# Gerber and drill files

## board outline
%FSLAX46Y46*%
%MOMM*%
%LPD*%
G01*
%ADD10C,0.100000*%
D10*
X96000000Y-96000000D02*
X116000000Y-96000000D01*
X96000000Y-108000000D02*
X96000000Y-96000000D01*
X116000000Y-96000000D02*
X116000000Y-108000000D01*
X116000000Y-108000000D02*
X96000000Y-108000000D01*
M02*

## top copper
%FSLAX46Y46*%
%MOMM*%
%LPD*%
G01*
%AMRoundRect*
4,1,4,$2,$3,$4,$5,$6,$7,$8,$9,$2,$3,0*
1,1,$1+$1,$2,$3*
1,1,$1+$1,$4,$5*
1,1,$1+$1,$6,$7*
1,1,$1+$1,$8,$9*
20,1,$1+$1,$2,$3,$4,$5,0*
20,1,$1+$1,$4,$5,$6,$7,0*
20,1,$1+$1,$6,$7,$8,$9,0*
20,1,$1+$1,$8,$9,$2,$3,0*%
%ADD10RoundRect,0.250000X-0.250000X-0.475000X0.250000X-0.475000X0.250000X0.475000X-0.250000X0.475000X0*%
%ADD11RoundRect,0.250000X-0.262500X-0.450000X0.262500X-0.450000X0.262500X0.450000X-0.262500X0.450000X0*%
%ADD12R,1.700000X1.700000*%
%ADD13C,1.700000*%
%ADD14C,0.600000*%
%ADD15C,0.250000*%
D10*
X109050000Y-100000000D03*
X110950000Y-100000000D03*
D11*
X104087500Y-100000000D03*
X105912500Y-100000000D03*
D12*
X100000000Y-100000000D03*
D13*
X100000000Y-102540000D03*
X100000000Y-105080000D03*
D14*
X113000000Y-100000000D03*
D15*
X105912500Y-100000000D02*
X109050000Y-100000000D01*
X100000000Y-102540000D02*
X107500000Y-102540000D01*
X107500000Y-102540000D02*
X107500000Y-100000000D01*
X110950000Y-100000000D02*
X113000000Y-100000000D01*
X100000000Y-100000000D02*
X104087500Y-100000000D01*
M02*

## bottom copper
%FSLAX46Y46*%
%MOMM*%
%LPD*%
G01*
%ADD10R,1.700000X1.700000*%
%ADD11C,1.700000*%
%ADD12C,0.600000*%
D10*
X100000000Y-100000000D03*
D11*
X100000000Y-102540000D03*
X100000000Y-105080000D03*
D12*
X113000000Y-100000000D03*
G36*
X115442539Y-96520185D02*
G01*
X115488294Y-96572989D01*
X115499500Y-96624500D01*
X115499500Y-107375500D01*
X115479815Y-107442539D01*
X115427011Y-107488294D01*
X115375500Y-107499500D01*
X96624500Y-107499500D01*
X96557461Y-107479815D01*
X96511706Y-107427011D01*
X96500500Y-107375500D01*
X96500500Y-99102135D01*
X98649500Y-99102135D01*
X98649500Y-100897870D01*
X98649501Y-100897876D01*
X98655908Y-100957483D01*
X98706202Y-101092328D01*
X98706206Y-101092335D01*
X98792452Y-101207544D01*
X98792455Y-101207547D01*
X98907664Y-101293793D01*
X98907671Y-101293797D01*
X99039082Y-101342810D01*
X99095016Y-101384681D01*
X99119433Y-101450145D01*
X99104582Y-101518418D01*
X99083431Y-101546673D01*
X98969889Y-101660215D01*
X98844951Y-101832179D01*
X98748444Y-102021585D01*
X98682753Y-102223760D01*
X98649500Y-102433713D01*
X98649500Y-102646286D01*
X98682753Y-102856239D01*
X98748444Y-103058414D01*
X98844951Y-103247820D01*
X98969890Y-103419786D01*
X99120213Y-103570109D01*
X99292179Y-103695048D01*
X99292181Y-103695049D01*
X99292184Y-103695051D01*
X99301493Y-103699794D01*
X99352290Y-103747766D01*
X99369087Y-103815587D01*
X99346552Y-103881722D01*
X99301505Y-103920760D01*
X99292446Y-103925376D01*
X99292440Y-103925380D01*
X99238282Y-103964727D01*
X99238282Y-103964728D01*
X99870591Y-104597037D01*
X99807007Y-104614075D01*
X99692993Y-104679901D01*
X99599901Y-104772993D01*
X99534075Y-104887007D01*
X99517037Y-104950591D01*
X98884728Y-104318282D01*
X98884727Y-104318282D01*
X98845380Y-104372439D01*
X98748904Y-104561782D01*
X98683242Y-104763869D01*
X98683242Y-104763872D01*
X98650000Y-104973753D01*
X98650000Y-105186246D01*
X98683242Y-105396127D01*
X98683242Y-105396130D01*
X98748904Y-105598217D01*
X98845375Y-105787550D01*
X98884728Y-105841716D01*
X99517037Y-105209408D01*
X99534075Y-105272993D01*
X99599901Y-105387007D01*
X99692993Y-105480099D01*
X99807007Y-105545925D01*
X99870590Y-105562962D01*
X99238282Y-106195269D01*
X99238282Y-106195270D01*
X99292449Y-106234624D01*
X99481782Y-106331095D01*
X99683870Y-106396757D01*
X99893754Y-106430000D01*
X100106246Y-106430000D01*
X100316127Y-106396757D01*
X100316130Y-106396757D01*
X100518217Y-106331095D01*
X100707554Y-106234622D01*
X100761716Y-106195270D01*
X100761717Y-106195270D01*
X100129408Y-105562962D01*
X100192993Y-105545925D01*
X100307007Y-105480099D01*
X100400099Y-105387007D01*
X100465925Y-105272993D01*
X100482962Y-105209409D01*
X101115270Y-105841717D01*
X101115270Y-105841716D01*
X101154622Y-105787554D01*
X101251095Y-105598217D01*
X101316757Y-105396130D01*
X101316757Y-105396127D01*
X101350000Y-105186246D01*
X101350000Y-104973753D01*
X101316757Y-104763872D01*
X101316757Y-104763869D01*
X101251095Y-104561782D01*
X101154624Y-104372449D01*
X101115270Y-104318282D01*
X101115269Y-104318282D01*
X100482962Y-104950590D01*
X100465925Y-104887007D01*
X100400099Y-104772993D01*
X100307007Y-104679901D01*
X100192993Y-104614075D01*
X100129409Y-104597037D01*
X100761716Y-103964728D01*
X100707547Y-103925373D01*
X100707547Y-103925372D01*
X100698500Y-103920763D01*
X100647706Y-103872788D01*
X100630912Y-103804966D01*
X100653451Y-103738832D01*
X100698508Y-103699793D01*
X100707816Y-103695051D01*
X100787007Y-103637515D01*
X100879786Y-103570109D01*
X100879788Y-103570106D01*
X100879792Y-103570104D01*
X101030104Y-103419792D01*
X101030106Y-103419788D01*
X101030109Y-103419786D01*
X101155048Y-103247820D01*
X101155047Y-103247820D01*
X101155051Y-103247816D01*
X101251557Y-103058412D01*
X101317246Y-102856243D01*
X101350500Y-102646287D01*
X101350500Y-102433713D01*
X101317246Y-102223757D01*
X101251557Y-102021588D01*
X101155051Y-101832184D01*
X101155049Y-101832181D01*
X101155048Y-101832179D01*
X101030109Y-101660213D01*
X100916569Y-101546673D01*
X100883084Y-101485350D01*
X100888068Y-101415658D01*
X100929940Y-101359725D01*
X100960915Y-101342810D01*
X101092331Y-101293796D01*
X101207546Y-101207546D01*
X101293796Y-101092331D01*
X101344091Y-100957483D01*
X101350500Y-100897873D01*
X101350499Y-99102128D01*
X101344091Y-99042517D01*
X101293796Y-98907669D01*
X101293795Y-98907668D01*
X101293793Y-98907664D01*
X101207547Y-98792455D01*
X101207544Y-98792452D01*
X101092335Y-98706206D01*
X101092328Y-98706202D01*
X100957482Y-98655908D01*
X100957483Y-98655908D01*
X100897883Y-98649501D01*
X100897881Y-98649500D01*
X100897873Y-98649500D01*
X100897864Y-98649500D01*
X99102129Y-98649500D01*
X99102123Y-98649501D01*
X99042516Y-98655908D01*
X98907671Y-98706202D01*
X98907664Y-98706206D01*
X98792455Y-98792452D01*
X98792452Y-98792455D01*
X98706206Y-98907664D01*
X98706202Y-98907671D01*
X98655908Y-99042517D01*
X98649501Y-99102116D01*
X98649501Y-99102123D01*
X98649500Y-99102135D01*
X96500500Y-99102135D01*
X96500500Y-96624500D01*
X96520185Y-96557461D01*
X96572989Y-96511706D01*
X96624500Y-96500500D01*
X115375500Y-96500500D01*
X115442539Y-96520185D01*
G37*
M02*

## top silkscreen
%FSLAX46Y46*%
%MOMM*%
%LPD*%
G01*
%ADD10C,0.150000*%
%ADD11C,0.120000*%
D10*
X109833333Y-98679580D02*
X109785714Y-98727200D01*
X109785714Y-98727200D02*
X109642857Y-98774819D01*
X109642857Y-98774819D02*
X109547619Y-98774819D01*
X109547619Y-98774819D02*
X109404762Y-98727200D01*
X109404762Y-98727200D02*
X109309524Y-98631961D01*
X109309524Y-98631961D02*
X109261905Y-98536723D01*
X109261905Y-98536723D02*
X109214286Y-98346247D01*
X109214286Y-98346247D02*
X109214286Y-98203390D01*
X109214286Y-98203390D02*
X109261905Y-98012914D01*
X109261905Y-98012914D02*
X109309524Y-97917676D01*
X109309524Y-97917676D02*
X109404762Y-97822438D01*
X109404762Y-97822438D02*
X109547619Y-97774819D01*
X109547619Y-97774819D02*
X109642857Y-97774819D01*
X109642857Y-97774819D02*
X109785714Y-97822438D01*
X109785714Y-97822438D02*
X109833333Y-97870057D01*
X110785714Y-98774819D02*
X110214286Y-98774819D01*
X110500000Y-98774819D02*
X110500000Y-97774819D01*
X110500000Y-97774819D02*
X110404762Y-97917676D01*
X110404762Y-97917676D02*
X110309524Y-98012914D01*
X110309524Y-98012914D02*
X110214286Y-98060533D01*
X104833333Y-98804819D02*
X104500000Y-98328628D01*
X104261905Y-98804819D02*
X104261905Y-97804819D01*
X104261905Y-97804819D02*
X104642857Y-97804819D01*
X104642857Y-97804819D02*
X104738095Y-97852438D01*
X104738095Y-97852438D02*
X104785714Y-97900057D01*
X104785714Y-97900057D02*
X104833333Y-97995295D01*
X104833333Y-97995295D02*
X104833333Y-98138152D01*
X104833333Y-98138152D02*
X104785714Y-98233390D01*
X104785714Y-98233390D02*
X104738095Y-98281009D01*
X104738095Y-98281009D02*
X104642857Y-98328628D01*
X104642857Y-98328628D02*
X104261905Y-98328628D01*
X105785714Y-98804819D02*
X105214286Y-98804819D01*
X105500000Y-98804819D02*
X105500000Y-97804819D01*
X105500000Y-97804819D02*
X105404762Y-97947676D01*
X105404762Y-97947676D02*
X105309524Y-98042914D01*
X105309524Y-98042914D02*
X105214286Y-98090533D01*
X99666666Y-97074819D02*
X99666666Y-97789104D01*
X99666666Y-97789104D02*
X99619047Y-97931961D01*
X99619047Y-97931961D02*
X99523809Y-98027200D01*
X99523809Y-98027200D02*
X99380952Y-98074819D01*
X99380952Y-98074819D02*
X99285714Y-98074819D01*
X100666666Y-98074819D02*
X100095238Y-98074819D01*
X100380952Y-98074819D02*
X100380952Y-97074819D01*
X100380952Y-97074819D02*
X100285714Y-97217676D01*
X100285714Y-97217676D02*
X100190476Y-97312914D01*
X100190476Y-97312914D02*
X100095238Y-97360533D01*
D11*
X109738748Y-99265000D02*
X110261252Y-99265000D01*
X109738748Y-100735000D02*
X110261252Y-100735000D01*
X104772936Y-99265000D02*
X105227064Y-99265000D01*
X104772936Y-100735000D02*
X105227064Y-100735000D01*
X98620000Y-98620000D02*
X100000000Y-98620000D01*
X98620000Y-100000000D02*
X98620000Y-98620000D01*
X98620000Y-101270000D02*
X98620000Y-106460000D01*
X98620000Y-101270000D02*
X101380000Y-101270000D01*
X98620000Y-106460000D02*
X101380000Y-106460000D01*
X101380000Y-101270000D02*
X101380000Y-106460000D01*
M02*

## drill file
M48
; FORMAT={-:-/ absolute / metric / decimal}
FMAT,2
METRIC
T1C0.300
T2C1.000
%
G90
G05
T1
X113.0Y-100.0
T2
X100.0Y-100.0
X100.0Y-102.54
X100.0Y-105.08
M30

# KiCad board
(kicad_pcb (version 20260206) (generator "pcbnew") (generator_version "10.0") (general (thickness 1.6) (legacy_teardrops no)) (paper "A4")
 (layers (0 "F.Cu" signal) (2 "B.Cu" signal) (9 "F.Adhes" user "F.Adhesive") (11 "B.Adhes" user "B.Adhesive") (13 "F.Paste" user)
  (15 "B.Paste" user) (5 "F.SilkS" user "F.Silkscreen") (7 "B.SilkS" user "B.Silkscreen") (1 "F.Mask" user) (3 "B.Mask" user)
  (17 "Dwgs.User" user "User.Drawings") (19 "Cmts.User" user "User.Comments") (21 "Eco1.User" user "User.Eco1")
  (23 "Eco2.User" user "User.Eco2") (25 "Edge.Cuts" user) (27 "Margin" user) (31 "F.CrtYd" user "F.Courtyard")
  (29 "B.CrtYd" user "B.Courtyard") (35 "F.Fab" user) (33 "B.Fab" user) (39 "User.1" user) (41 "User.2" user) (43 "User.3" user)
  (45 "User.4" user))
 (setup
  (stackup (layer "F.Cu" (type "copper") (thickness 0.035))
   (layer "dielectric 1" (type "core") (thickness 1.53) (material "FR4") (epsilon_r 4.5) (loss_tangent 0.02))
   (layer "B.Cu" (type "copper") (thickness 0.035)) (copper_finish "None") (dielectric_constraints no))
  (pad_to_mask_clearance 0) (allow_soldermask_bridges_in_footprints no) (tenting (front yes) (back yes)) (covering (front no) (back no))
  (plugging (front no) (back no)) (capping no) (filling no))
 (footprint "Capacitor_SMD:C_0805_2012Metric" (layer "F.Cu") (at 110 100)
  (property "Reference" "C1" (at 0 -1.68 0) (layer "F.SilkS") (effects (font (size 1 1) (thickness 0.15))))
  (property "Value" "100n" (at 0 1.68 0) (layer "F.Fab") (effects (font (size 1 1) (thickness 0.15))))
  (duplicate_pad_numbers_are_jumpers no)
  (fp_line (start -0.261252 -0.735) (end 0.261252 -0.735) (stroke (width 0.12) (type solid)) (layer "F.SilkS"))
  (fp_line (start -0.261252 0.735) (end 0.261252 0.735) (stroke (width 0.12) (type solid)) (layer "F.SilkS"))
  (pad "1" smd roundrect (at -0.95 0) (size 1 1.45) (layers "F.Cu" "F.Mask" "F.Paste") (roundrect_rratio 0.25) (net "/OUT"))
  (pad "2" smd roundrect (at 0.95 0) (size 1 1.45) (layers "F.Cu" "F.Mask" "F.Paste") (roundrect_rratio 0.25) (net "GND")))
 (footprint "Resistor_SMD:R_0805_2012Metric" (layer "F.Cu") (at 105 100)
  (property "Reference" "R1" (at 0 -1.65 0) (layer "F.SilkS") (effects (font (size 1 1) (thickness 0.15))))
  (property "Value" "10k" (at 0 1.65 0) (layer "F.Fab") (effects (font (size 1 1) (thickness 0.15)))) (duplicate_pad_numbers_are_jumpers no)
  (fp_line (start -0.227064 -0.735) (end 0.227064 -0.735) (stroke (width 0.12) (type solid)) (layer "F.SilkS"))
  (fp_line (start -0.227064 0.735) (end 0.227064 0.735) (stroke (width 0.12) (type solid)) (layer "F.SilkS"))
  (pad "1" smd roundrect (at -0.9125 0) (size 1.025 1.4) (layers "F.Cu" "F.Mask" "F.Paste") (roundrect_rratio 0.243902) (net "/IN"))
  (pad "2" smd roundrect (at 0.9125 0) (size 1.025 1.4) (layers "F.Cu" "F.Mask" "F.Paste") (roundrect_rratio 0.243902) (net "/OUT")))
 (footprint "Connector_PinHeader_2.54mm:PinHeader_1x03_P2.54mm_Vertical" (layer "F.Cu") (at 100 100)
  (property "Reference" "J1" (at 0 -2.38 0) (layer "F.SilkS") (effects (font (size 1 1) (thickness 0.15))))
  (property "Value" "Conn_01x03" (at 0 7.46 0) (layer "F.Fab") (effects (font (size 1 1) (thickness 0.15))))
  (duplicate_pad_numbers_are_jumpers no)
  (fp_line (start -1.38 -1.38) (end 0 -1.38) (stroke (width 0.12) (type solid)) (layer "F.SilkS"))
  (fp_line (start -1.38 0) (end -1.38 -1.38) (stroke (width 0.12) (type solid)) (layer "F.SilkS"))
  (fp_line (start -1.38 1.27) (end -1.38 6.46) (stroke (width 0.12) (type solid)) (layer "F.SilkS"))
  (fp_line (start -1.38 1.27) (end 1.38 1.27) (stroke (width 0.12) (type solid)) (layer "F.SilkS"))
  (fp_line (start -1.38 6.46) (end 1.38 6.46) (stroke (width 0.12) (type solid)) (layer "F.SilkS"))
  (fp_line (start 1.38 1.27) (end 1.38 6.46) (stroke (width 0.12) (type solid)) (layer "F.SilkS"))
  (pad "1" thru_hole rect (at 0 0) (size 1.7 1.7) (drill 1) (layers "*.Cu" "*.Mask") (remove_unused_layers no) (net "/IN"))
  (pad "2" thru_hole circle (at 0 2.54) (size 1.7 1.7) (drill 1) (layers "*.Cu" "*.Mask") (remove_unused_layers no) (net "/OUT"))
  (pad "3" thru_hole circle (at 0 5.08) (size 1.7 1.7) (drill 1) (layers "*.Cu" "*.Mask") (remove_unused_layers no) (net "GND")))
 (gr_line (start 96 96) (end 116 96) (stroke (width 0.1) (type default)) (layer "Edge.Cuts"))
 (gr_line (start 96 108) (end 96 96) (stroke (width 0.1) (type default)) (layer "Edge.Cuts"))
 (gr_line (start 116 96) (end 116 108) (stroke (width 0.1) (type default)) (layer "Edge.Cuts"))
 (gr_line (start 116 108) (end 96 108) (stroke (width 0.1) (type default)) (layer "Edge.Cuts"))
 (segment (start 105.9125 100) (end 109.05 100) (width 0.25) (layer "F.Cu") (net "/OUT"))
 (segment (start 100 102.54) (end 107.5 102.54) (width 0.25) (layer "F.Cu") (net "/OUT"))
 (segment (start 107.5 102.54) (end 107.5 100) (width 0.25) (layer "F.Cu") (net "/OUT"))
 (segment (start 110.95 100) (end 113 100) (width 0.25) (layer "F.Cu") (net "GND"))
 (via (at 113 100) (size 0.6) (drill 0.3) (layers "F.Cu" "B.Cu") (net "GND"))
 (segment (start 100 100) (end 104.0875 100) (width 0.25) (layer "F.Cu") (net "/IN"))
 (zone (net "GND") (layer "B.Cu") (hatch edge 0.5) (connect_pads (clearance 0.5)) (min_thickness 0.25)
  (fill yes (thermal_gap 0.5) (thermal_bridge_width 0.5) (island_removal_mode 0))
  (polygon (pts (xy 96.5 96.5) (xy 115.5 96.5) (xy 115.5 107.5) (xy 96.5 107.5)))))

